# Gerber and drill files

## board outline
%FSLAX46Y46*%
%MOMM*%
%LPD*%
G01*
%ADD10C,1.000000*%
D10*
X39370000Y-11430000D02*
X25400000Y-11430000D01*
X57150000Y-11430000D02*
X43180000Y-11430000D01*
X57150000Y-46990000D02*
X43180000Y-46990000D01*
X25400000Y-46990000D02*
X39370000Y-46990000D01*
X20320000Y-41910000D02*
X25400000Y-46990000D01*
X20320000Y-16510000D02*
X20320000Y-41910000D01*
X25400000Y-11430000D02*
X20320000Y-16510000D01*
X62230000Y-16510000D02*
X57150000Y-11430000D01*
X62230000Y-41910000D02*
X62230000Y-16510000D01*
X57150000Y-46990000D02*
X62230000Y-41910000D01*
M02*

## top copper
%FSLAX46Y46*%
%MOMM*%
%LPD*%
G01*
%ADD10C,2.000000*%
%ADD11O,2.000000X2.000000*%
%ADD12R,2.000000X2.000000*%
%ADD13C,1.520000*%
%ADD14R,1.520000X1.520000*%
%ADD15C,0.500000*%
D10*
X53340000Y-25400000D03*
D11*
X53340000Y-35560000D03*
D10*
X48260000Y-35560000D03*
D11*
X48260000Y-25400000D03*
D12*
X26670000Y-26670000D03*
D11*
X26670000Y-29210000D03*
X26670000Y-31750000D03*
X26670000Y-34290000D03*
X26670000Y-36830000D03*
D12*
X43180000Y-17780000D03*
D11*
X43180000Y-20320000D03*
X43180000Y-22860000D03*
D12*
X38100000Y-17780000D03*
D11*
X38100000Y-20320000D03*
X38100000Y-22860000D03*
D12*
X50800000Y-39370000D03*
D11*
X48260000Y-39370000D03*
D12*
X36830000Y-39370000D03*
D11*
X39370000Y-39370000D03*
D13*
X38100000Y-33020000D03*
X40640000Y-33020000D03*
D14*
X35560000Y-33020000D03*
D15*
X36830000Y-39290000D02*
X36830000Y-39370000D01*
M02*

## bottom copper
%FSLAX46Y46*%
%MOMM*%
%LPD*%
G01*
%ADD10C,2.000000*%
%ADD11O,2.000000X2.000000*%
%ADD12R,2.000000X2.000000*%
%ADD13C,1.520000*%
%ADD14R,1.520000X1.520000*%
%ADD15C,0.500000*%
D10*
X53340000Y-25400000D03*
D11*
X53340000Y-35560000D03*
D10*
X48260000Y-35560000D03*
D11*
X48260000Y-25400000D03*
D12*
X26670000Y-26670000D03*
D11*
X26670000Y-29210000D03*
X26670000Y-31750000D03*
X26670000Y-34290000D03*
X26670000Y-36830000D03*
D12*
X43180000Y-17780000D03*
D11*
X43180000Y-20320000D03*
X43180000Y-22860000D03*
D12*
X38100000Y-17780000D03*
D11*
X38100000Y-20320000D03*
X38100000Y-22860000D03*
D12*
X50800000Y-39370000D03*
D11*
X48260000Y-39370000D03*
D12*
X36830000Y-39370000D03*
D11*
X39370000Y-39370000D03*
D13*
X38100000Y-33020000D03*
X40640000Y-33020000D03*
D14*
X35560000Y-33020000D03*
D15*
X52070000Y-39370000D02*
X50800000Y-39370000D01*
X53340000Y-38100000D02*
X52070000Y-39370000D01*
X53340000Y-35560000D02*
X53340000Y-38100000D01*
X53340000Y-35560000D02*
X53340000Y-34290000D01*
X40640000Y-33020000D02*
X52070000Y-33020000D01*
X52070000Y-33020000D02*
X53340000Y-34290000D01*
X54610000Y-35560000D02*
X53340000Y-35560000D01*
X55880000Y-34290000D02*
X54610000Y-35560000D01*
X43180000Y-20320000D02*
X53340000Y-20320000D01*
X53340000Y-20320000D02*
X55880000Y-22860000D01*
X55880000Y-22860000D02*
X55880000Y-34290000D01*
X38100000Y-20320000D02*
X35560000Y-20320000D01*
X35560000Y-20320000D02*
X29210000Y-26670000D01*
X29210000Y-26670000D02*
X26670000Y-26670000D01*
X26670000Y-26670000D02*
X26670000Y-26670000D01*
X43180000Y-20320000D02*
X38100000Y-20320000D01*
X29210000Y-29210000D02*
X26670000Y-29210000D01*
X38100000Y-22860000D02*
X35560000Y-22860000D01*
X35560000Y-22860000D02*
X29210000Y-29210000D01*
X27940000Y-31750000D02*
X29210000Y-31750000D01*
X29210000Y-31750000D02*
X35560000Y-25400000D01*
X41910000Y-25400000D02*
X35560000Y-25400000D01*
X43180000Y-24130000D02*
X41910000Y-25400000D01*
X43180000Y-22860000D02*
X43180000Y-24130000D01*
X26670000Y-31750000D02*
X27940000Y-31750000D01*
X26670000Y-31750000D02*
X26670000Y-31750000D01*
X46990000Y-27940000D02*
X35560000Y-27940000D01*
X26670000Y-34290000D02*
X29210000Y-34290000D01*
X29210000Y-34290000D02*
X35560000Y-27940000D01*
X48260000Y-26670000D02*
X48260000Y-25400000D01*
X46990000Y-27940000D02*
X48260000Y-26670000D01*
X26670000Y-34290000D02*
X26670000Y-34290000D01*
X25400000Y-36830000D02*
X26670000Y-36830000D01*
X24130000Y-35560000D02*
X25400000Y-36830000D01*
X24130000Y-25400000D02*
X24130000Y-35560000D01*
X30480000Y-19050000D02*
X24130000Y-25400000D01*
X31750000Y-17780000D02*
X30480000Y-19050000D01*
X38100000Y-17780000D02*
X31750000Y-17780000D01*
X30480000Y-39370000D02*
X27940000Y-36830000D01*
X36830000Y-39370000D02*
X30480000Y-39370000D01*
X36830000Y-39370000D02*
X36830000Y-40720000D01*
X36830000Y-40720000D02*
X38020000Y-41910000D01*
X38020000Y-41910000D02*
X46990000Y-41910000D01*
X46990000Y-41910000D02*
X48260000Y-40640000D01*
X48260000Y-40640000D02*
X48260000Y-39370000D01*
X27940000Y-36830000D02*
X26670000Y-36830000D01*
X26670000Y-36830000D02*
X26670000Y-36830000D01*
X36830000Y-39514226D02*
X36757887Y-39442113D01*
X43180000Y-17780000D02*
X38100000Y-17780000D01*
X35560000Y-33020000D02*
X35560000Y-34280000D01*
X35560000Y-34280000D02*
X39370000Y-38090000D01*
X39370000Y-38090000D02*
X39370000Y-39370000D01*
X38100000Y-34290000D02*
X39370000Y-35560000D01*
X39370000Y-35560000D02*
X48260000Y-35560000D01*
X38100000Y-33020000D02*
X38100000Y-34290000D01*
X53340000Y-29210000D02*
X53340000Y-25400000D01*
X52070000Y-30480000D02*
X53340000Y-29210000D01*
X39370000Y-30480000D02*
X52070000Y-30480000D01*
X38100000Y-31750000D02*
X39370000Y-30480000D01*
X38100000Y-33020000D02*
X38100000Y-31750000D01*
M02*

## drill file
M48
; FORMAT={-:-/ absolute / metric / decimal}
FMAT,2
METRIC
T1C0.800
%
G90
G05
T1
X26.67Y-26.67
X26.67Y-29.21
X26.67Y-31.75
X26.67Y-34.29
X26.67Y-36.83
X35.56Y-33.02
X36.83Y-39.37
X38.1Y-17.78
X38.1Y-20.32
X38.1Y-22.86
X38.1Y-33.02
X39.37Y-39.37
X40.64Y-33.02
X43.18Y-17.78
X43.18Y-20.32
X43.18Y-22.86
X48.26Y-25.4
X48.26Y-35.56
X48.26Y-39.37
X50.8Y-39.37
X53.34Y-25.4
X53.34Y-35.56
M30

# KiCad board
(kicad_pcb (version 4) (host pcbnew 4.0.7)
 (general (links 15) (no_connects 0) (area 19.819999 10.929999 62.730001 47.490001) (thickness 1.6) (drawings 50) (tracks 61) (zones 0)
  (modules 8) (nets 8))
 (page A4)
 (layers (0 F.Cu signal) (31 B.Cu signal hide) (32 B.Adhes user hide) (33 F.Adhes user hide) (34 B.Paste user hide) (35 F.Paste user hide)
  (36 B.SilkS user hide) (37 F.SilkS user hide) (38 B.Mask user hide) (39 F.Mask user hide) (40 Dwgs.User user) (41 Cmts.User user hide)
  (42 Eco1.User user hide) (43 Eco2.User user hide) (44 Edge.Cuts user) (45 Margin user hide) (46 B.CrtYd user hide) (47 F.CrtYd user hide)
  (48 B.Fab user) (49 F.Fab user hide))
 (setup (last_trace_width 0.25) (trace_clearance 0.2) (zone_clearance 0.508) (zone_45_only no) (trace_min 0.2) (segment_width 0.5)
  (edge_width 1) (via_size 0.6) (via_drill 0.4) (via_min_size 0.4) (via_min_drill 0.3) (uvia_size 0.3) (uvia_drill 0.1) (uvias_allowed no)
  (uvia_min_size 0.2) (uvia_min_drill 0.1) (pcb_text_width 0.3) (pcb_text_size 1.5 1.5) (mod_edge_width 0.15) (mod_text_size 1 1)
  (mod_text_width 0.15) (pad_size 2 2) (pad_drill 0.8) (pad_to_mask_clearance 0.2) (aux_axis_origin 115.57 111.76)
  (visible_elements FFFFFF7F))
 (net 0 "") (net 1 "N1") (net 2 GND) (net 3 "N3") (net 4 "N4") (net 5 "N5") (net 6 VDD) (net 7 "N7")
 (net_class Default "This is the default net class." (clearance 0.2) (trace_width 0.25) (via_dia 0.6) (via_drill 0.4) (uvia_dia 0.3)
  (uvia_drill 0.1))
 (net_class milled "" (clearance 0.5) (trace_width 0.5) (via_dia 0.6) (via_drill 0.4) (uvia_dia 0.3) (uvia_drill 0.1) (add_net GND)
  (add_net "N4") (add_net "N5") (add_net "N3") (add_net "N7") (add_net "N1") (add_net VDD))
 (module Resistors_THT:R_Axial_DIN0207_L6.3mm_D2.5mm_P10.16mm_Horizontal (layer F.Cu) (at 53.34 25.4 270)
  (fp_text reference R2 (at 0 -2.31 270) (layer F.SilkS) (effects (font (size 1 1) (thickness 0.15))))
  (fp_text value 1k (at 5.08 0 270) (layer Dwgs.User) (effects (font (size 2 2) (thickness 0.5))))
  (pad 1 thru_hole circle (at 0 0 270) (size 2 2) (drill 0.8) (layers *.Cu *.Mask) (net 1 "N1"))
  (pad 2 thru_hole oval (at 10.16 0 270) (size 2 2) (drill 0.8) (layers *.Cu *.Mask) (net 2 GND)))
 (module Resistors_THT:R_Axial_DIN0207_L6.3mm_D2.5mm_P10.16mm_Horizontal (layer F.Cu) (at 48.26 35.56 90)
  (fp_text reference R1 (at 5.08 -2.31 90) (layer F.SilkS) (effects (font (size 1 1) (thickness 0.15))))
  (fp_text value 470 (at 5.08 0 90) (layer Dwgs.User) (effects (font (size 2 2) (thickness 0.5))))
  (pad 1 thru_hole circle (at 0 0 90) (size 2 2) (drill 0.8) (layers *.Cu *.Mask) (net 1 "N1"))
  (pad 2 thru_hole oval (at 10.16 0 90) (size 2 2) (drill 0.8) (layers *.Cu *.Mask) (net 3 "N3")))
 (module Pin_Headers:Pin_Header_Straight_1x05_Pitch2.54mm (layer F.Cu) (at 26.67 26.67)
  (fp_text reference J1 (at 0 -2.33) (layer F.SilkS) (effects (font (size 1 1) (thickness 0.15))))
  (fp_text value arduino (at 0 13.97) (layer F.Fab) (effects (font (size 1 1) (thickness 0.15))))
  (pad 1 thru_hole rect (at 0 0) (size 2 2) (drill 0.8) (layers *.Cu *.Mask) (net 2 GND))
  (pad 2 thru_hole oval (at 0 2.54) (size 2 2) (drill 0.8) (layers *.Cu *.Mask) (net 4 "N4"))
  (pad 3 thru_hole oval (at 0 5.08) (size 2 2) (drill 0.8) (layers *.Cu *.Mask) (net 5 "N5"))
  (pad 4 thru_hole oval (at 0 7.62) (size 2 2) (drill 0.8) (layers *.Cu *.Mask) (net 3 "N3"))
  (pad 5 thru_hole oval (at 0 10.16) (size 2 2) (drill 0.8) (layers *.Cu *.Mask) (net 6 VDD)))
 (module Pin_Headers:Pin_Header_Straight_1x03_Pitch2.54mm (layer F.Cu) (at 43.18 17.78)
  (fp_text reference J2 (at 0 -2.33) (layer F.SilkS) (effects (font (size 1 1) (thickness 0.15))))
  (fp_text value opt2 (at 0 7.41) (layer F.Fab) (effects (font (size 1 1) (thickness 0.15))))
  (pad 1 thru_hole rect (at 0 0) (size 2 2) (drill 0.8) (layers *.Cu *.Mask) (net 6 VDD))
  (pad 2 thru_hole oval (at 0 2.54) (size 2 2) (drill 0.8) (layers *.Cu *.Mask) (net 2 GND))
  (pad 3 thru_hole oval (at 0 5.08) (size 2 2) (drill 0.8) (layers *.Cu *.Mask) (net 5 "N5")))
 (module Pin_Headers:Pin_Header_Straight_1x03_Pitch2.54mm (layer F.Cu) (at 38.1 17.78)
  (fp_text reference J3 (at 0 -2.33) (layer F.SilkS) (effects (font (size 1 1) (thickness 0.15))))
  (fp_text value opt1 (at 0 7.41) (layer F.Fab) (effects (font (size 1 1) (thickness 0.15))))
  (pad 1 thru_hole rect (at 0 0) (size 2 2) (drill 0.8) (layers *.Cu *.Mask) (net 6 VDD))
  (pad 2 thru_hole oval (at 0 2.54) (size 2 2) (drill 0.8) (layers *.Cu *.Mask) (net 2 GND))
  (pad 3 thru_hole oval (at 0 5.08) (size 2 2) (drill 0.8) (layers *.Cu *.Mask) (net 4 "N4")))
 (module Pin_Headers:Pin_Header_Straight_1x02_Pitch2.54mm (layer F.Cu) (at 50.8 39.37 270)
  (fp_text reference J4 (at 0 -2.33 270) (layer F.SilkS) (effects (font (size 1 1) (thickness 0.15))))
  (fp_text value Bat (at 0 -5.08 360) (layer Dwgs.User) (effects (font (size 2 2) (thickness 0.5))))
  (pad 1 thru_hole rect (at 0 0 270) (size 2 2) (drill 0.8) (layers *.Cu *.Mask) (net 2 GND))
  (pad 2 thru_hole oval (at 0 2.54 270) (size 2 2) (drill 0.8) (layers *.Cu *.Mask) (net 6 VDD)))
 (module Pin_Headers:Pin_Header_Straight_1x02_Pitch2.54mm (layer F.Cu) (at 36.83 39.37 90)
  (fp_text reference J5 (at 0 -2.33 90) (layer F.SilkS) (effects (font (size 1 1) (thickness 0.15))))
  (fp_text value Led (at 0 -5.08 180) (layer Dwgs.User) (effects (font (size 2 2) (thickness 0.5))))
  (pad 1 thru_hole rect (at 0 0 90) (size 2 2) (drill 0.8) (layers *.Cu *.Mask) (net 6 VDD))
  (pad 2 thru_hole oval (at 0 2.54 90) (size 2 2) (drill 0.8) (layers *.Cu *.Mask) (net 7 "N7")))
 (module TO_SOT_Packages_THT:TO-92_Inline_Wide (layer F.Cu) (at 35.56 33.02)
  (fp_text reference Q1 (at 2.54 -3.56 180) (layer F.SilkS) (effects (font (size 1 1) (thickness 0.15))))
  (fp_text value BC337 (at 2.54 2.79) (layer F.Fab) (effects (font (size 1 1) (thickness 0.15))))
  (pad 2 thru_hole circle (at 2.54 0 90) (size 1.52 1.52) (drill 0.8) (layers *.Cu *.Mask) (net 1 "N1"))
  (pad 3 thru_hole circle (at 5.08 0 90) (size 1.52 1.52) (drill 0.8) (layers *.Cu *.Mask) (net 2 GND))
  (pad 1 thru_hole rect (at 0 0 90) (size 1.52 1.52) (drill 0.8) (layers *.Cu *.Mask) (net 7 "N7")))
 (gr_line (start 39.37 11.43) (end 25.4 11.43) (layer Edge.Cuts) (width 1))
 (gr_line (start 57.15 11.43) (end 43.18 11.43) (layer Edge.Cuts) (width 1))
 (gr_line (start 57.15 46.99) (end 43.18 46.99) (layer Edge.Cuts) (width 1))
 (gr_line (start 25.4 46.99) (end 39.37 46.99) (layer Edge.Cuts) (width 1))
 (gr_line (start 20.32 41.91) (end 25.4 46.99) (layer Edge.Cuts) (width 1))
 (gr_line (start 20.32 16.51) (end 20.32 41.91) (layer Edge.Cuts) (width 1))
 (gr_line (start 25.4 11.43) (end 20.32 16.51) (layer Edge.Cuts) (width 1))
 (gr_line (start 62.23 16.51) (end 57.15 11.43) (layer Edge.Cuts) (width 1))
 (gr_line (start 62.23 41.91) (end 62.23 16.51) (layer Edge.Cuts) (width 1))
 (gr_line (start 57.15 46.99) (end 62.23 41.91) (layer Edge.Cuts) (width 1))
 (segment (start 52.07 39.37) (end 50.8 39.37) (width 0.5) (layer B.Cu) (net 2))
 (segment (start 53.34 38.1) (end 52.07 39.37) (width 0.5) (layer B.Cu) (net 2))
 (segment (start 53.34 35.56) (end 53.34 38.1) (width 0.5) (layer B.Cu) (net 2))
 (segment (start 53.34 35.56) (end 53.34 34.29) (width 0.5) (layer B.Cu) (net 2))
 (segment (start 40.64 33.02) (end 52.07 33.02) (width 0.5) (layer B.Cu) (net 2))
 (segment (start 52.07 33.02) (end 53.34 34.29) (width 0.5) (layer B.Cu) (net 2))
 (segment (start 54.61 35.56) (end 53.34 35.56) (width 0.5) (layer B.Cu) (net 2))
 (segment (start 55.88 34.29) (end 54.61 35.56) (width 0.5) (layer B.Cu) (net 2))
 (segment (start 43.18 20.32) (end 53.34 20.32) (width 0.5) (layer B.Cu) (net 2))
 (segment (start 53.34 20.32) (end 55.88 22.86) (width 0.5) (layer B.Cu) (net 2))
 (segment (start 55.88 22.86) (end 55.88 34.29) (width 0.5) (layer B.Cu) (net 2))
 (segment (start 38.1 20.32) (end 35.56 20.32) (width 0.5) (layer B.Cu) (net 2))
 (segment (start 35.56 20.32) (end 29.21 26.67) (width 0.5) (layer B.Cu) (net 2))
 (segment (start 29.21 26.67) (end 26.67 26.67) (width 0.5) (layer B.Cu) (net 2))
 (segment (start 26.67 26.67) (end 26.67 26.67) (width 0.5) (layer B.Cu) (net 2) (status 30))
 (segment (start 43.18 20.32) (end 38.1 20.32) (width 0.5) (layer B.Cu) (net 2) (status 20))
 (segment (start 29.21 29.21) (end 26.67 29.21) (width 0.5) (layer B.Cu) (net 4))
 (segment (start 38.1 22.86) (end 35.56 22.86) (width 0.5) (layer B.Cu) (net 4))
 (segment (start 35.56 22.86) (end 29.21 29.21) (width 0.5) (layer B.Cu) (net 4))
 (segment (start 27.94 31.75) (end 29.21 31.75) (width 0.5) (layer B.Cu) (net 5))
 (segment (start 29.21 31.75) (end 35.56 25.4) (width 0.5) (layer B.Cu) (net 5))
 (segment (start 41.91 25.4) (end 35.56 25.4) (width 0.5) (layer B.Cu) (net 5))
 (segment (start 43.18 24.13) (end 41.91 25.4) (width 0.5) (layer B.Cu) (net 5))
 (segment (start 43.18 22.86) (end 43.18 24.13) (width 0.5) (layer B.Cu) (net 5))
 (segment (start 26.67 31.75) (end 27.94 31.75) (width 0.5) (layer B.Cu) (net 5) (status 10))
 (segment (start 26.67 31.75) (end 26.67 31.75) (width 0.5) (layer B.Cu) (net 5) (status 30))
 (segment (start 46.99 27.94) (end 35.56 27.94) (width 0.5) (layer B.Cu) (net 3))
 (segment (start 26.67 34.29) (end 29.21 34.29) (width 0.5) (layer B.Cu) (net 3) (status 10))
 (segment (start 29.21 34.29) (end 35.56 27.94) (width 0.5) (layer B.Cu) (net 3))
 (segment (start 48.26 26.67) (end 48.26 25.4) (width 0.5) (layer B.Cu) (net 3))
 (segment (start 46.99 27.94) (end 48.26 26.67) (width 0.5) (layer B.Cu) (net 3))
 (segment (start 26.67 34.29) (end 26.67 34.29) (width 0.5) (layer B.Cu) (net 3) (status 30))
 (segment (start 25.4 36.83) (end 26.67 36.83) (width 0.5) (layer B.Cu) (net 6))
 (segment (start 24.13 35.56) (end 25.4 36.83) (width 0.5) (layer B.Cu) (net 6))
 (segment (start 24.13 25.4) (end 24.13 35.56) (width 0.5) (layer B.Cu) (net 6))
 (segment (start 30.48 19.05) (end 24.13 25.4) (width 0.5) (layer B.Cu) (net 6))
 (segment (start 31.75 17.78) (end 30.48 19.05) (width 0.5) (layer B.Cu) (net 6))
 (segment (start 38.1 17.78) (end 31.75 17.78) (width 0.5) (layer B.Cu) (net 6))
 (segment (start 30.48 39.37) (end 27.94 36.83) (width 0.5) (layer B.Cu) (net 6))
 (segment (start 36.83 39.37) (end 30.48 39.37) (width 0.5) (layer B.Cu) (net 6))
 (segment (start 36.83 39.37) (end 36.83 40.72) (width 0.5) (layer B.Cu) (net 6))
 (segment (start 36.83 40.72) (end 38.02 41.91) (width 0.5) (layer B.Cu) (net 6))
 (segment (start 38.02 41.91) (end 46.99 41.91) (width 0.5) (layer B.Cu) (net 6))
 (segment (start 46.99 41.91) (end 48.26 40.64) (width 0.5) (layer B.Cu) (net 6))
 (segment (start 48.26 40.64) (end 48.26 39.37) (width 0.5) (layer B.Cu) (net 6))
 (segment (start 27.94 36.83) (end 26.67 36.83) (width 0.5) (layer B.Cu) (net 6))
 (segment (start 26.67 36.83) (end 26.67 36.83) (width 0.5) (layer B.Cu) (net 6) (status 20))
 (segment (start 36.83 39.514226) (end 36.757887 39.442113) (width 0.5) (layer B.Cu) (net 6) (status 30))
 (segment (start 36.83 39.29) (end 36.83 39.37) (width 0.5) (layer F.Cu) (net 6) (status 30))
 (segment (start 43.18 17.78) (end 38.1 17.78) (width 0.5) (layer B.Cu) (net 6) (status 20))
 (segment (start 35.56 33.02) (end 35.56 34.28) (width 0.5) (layer B.Cu) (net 7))
 (segment (start 35.56 34.28) (end 39.37 38.09) (width 0.5) (layer B.Cu) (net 7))
 (segment (start 39.37 38.09) (end 39.37 39.37) (width 0.5) (layer B.Cu) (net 7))
 (segment (start 38.1 34.29) (end 39.37 35.56) (width 0.5) (layer B.Cu) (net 1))
 (segment (start 39.37 35.56) (end 48.26 35.56) (width 0.5) (layer B.Cu) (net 1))
 (segment (start 38.1 33.02) (end 38.1 34.29) (width 0.5) (layer B.Cu) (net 1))
 (segment (start 53.34 29.21) (end 53.34 25.4) (width 0.5) (layer B.Cu) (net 1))
 (segment (start 52.07 30.48) (end 53.34 29.21) (width 0.5) (layer B.Cu) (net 1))
 (segment (start 39.37 30.48) (end 52.07 30.48) (width 0.5) (layer B.Cu) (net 1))
 (segment (start 38.1 31.75) (end 39.37 30.48) (width 0.5) (layer B.Cu) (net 1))
 (segment (start 38.1 33.02) (end 38.1 31.75) (width 0.5) (layer B.Cu) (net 1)))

